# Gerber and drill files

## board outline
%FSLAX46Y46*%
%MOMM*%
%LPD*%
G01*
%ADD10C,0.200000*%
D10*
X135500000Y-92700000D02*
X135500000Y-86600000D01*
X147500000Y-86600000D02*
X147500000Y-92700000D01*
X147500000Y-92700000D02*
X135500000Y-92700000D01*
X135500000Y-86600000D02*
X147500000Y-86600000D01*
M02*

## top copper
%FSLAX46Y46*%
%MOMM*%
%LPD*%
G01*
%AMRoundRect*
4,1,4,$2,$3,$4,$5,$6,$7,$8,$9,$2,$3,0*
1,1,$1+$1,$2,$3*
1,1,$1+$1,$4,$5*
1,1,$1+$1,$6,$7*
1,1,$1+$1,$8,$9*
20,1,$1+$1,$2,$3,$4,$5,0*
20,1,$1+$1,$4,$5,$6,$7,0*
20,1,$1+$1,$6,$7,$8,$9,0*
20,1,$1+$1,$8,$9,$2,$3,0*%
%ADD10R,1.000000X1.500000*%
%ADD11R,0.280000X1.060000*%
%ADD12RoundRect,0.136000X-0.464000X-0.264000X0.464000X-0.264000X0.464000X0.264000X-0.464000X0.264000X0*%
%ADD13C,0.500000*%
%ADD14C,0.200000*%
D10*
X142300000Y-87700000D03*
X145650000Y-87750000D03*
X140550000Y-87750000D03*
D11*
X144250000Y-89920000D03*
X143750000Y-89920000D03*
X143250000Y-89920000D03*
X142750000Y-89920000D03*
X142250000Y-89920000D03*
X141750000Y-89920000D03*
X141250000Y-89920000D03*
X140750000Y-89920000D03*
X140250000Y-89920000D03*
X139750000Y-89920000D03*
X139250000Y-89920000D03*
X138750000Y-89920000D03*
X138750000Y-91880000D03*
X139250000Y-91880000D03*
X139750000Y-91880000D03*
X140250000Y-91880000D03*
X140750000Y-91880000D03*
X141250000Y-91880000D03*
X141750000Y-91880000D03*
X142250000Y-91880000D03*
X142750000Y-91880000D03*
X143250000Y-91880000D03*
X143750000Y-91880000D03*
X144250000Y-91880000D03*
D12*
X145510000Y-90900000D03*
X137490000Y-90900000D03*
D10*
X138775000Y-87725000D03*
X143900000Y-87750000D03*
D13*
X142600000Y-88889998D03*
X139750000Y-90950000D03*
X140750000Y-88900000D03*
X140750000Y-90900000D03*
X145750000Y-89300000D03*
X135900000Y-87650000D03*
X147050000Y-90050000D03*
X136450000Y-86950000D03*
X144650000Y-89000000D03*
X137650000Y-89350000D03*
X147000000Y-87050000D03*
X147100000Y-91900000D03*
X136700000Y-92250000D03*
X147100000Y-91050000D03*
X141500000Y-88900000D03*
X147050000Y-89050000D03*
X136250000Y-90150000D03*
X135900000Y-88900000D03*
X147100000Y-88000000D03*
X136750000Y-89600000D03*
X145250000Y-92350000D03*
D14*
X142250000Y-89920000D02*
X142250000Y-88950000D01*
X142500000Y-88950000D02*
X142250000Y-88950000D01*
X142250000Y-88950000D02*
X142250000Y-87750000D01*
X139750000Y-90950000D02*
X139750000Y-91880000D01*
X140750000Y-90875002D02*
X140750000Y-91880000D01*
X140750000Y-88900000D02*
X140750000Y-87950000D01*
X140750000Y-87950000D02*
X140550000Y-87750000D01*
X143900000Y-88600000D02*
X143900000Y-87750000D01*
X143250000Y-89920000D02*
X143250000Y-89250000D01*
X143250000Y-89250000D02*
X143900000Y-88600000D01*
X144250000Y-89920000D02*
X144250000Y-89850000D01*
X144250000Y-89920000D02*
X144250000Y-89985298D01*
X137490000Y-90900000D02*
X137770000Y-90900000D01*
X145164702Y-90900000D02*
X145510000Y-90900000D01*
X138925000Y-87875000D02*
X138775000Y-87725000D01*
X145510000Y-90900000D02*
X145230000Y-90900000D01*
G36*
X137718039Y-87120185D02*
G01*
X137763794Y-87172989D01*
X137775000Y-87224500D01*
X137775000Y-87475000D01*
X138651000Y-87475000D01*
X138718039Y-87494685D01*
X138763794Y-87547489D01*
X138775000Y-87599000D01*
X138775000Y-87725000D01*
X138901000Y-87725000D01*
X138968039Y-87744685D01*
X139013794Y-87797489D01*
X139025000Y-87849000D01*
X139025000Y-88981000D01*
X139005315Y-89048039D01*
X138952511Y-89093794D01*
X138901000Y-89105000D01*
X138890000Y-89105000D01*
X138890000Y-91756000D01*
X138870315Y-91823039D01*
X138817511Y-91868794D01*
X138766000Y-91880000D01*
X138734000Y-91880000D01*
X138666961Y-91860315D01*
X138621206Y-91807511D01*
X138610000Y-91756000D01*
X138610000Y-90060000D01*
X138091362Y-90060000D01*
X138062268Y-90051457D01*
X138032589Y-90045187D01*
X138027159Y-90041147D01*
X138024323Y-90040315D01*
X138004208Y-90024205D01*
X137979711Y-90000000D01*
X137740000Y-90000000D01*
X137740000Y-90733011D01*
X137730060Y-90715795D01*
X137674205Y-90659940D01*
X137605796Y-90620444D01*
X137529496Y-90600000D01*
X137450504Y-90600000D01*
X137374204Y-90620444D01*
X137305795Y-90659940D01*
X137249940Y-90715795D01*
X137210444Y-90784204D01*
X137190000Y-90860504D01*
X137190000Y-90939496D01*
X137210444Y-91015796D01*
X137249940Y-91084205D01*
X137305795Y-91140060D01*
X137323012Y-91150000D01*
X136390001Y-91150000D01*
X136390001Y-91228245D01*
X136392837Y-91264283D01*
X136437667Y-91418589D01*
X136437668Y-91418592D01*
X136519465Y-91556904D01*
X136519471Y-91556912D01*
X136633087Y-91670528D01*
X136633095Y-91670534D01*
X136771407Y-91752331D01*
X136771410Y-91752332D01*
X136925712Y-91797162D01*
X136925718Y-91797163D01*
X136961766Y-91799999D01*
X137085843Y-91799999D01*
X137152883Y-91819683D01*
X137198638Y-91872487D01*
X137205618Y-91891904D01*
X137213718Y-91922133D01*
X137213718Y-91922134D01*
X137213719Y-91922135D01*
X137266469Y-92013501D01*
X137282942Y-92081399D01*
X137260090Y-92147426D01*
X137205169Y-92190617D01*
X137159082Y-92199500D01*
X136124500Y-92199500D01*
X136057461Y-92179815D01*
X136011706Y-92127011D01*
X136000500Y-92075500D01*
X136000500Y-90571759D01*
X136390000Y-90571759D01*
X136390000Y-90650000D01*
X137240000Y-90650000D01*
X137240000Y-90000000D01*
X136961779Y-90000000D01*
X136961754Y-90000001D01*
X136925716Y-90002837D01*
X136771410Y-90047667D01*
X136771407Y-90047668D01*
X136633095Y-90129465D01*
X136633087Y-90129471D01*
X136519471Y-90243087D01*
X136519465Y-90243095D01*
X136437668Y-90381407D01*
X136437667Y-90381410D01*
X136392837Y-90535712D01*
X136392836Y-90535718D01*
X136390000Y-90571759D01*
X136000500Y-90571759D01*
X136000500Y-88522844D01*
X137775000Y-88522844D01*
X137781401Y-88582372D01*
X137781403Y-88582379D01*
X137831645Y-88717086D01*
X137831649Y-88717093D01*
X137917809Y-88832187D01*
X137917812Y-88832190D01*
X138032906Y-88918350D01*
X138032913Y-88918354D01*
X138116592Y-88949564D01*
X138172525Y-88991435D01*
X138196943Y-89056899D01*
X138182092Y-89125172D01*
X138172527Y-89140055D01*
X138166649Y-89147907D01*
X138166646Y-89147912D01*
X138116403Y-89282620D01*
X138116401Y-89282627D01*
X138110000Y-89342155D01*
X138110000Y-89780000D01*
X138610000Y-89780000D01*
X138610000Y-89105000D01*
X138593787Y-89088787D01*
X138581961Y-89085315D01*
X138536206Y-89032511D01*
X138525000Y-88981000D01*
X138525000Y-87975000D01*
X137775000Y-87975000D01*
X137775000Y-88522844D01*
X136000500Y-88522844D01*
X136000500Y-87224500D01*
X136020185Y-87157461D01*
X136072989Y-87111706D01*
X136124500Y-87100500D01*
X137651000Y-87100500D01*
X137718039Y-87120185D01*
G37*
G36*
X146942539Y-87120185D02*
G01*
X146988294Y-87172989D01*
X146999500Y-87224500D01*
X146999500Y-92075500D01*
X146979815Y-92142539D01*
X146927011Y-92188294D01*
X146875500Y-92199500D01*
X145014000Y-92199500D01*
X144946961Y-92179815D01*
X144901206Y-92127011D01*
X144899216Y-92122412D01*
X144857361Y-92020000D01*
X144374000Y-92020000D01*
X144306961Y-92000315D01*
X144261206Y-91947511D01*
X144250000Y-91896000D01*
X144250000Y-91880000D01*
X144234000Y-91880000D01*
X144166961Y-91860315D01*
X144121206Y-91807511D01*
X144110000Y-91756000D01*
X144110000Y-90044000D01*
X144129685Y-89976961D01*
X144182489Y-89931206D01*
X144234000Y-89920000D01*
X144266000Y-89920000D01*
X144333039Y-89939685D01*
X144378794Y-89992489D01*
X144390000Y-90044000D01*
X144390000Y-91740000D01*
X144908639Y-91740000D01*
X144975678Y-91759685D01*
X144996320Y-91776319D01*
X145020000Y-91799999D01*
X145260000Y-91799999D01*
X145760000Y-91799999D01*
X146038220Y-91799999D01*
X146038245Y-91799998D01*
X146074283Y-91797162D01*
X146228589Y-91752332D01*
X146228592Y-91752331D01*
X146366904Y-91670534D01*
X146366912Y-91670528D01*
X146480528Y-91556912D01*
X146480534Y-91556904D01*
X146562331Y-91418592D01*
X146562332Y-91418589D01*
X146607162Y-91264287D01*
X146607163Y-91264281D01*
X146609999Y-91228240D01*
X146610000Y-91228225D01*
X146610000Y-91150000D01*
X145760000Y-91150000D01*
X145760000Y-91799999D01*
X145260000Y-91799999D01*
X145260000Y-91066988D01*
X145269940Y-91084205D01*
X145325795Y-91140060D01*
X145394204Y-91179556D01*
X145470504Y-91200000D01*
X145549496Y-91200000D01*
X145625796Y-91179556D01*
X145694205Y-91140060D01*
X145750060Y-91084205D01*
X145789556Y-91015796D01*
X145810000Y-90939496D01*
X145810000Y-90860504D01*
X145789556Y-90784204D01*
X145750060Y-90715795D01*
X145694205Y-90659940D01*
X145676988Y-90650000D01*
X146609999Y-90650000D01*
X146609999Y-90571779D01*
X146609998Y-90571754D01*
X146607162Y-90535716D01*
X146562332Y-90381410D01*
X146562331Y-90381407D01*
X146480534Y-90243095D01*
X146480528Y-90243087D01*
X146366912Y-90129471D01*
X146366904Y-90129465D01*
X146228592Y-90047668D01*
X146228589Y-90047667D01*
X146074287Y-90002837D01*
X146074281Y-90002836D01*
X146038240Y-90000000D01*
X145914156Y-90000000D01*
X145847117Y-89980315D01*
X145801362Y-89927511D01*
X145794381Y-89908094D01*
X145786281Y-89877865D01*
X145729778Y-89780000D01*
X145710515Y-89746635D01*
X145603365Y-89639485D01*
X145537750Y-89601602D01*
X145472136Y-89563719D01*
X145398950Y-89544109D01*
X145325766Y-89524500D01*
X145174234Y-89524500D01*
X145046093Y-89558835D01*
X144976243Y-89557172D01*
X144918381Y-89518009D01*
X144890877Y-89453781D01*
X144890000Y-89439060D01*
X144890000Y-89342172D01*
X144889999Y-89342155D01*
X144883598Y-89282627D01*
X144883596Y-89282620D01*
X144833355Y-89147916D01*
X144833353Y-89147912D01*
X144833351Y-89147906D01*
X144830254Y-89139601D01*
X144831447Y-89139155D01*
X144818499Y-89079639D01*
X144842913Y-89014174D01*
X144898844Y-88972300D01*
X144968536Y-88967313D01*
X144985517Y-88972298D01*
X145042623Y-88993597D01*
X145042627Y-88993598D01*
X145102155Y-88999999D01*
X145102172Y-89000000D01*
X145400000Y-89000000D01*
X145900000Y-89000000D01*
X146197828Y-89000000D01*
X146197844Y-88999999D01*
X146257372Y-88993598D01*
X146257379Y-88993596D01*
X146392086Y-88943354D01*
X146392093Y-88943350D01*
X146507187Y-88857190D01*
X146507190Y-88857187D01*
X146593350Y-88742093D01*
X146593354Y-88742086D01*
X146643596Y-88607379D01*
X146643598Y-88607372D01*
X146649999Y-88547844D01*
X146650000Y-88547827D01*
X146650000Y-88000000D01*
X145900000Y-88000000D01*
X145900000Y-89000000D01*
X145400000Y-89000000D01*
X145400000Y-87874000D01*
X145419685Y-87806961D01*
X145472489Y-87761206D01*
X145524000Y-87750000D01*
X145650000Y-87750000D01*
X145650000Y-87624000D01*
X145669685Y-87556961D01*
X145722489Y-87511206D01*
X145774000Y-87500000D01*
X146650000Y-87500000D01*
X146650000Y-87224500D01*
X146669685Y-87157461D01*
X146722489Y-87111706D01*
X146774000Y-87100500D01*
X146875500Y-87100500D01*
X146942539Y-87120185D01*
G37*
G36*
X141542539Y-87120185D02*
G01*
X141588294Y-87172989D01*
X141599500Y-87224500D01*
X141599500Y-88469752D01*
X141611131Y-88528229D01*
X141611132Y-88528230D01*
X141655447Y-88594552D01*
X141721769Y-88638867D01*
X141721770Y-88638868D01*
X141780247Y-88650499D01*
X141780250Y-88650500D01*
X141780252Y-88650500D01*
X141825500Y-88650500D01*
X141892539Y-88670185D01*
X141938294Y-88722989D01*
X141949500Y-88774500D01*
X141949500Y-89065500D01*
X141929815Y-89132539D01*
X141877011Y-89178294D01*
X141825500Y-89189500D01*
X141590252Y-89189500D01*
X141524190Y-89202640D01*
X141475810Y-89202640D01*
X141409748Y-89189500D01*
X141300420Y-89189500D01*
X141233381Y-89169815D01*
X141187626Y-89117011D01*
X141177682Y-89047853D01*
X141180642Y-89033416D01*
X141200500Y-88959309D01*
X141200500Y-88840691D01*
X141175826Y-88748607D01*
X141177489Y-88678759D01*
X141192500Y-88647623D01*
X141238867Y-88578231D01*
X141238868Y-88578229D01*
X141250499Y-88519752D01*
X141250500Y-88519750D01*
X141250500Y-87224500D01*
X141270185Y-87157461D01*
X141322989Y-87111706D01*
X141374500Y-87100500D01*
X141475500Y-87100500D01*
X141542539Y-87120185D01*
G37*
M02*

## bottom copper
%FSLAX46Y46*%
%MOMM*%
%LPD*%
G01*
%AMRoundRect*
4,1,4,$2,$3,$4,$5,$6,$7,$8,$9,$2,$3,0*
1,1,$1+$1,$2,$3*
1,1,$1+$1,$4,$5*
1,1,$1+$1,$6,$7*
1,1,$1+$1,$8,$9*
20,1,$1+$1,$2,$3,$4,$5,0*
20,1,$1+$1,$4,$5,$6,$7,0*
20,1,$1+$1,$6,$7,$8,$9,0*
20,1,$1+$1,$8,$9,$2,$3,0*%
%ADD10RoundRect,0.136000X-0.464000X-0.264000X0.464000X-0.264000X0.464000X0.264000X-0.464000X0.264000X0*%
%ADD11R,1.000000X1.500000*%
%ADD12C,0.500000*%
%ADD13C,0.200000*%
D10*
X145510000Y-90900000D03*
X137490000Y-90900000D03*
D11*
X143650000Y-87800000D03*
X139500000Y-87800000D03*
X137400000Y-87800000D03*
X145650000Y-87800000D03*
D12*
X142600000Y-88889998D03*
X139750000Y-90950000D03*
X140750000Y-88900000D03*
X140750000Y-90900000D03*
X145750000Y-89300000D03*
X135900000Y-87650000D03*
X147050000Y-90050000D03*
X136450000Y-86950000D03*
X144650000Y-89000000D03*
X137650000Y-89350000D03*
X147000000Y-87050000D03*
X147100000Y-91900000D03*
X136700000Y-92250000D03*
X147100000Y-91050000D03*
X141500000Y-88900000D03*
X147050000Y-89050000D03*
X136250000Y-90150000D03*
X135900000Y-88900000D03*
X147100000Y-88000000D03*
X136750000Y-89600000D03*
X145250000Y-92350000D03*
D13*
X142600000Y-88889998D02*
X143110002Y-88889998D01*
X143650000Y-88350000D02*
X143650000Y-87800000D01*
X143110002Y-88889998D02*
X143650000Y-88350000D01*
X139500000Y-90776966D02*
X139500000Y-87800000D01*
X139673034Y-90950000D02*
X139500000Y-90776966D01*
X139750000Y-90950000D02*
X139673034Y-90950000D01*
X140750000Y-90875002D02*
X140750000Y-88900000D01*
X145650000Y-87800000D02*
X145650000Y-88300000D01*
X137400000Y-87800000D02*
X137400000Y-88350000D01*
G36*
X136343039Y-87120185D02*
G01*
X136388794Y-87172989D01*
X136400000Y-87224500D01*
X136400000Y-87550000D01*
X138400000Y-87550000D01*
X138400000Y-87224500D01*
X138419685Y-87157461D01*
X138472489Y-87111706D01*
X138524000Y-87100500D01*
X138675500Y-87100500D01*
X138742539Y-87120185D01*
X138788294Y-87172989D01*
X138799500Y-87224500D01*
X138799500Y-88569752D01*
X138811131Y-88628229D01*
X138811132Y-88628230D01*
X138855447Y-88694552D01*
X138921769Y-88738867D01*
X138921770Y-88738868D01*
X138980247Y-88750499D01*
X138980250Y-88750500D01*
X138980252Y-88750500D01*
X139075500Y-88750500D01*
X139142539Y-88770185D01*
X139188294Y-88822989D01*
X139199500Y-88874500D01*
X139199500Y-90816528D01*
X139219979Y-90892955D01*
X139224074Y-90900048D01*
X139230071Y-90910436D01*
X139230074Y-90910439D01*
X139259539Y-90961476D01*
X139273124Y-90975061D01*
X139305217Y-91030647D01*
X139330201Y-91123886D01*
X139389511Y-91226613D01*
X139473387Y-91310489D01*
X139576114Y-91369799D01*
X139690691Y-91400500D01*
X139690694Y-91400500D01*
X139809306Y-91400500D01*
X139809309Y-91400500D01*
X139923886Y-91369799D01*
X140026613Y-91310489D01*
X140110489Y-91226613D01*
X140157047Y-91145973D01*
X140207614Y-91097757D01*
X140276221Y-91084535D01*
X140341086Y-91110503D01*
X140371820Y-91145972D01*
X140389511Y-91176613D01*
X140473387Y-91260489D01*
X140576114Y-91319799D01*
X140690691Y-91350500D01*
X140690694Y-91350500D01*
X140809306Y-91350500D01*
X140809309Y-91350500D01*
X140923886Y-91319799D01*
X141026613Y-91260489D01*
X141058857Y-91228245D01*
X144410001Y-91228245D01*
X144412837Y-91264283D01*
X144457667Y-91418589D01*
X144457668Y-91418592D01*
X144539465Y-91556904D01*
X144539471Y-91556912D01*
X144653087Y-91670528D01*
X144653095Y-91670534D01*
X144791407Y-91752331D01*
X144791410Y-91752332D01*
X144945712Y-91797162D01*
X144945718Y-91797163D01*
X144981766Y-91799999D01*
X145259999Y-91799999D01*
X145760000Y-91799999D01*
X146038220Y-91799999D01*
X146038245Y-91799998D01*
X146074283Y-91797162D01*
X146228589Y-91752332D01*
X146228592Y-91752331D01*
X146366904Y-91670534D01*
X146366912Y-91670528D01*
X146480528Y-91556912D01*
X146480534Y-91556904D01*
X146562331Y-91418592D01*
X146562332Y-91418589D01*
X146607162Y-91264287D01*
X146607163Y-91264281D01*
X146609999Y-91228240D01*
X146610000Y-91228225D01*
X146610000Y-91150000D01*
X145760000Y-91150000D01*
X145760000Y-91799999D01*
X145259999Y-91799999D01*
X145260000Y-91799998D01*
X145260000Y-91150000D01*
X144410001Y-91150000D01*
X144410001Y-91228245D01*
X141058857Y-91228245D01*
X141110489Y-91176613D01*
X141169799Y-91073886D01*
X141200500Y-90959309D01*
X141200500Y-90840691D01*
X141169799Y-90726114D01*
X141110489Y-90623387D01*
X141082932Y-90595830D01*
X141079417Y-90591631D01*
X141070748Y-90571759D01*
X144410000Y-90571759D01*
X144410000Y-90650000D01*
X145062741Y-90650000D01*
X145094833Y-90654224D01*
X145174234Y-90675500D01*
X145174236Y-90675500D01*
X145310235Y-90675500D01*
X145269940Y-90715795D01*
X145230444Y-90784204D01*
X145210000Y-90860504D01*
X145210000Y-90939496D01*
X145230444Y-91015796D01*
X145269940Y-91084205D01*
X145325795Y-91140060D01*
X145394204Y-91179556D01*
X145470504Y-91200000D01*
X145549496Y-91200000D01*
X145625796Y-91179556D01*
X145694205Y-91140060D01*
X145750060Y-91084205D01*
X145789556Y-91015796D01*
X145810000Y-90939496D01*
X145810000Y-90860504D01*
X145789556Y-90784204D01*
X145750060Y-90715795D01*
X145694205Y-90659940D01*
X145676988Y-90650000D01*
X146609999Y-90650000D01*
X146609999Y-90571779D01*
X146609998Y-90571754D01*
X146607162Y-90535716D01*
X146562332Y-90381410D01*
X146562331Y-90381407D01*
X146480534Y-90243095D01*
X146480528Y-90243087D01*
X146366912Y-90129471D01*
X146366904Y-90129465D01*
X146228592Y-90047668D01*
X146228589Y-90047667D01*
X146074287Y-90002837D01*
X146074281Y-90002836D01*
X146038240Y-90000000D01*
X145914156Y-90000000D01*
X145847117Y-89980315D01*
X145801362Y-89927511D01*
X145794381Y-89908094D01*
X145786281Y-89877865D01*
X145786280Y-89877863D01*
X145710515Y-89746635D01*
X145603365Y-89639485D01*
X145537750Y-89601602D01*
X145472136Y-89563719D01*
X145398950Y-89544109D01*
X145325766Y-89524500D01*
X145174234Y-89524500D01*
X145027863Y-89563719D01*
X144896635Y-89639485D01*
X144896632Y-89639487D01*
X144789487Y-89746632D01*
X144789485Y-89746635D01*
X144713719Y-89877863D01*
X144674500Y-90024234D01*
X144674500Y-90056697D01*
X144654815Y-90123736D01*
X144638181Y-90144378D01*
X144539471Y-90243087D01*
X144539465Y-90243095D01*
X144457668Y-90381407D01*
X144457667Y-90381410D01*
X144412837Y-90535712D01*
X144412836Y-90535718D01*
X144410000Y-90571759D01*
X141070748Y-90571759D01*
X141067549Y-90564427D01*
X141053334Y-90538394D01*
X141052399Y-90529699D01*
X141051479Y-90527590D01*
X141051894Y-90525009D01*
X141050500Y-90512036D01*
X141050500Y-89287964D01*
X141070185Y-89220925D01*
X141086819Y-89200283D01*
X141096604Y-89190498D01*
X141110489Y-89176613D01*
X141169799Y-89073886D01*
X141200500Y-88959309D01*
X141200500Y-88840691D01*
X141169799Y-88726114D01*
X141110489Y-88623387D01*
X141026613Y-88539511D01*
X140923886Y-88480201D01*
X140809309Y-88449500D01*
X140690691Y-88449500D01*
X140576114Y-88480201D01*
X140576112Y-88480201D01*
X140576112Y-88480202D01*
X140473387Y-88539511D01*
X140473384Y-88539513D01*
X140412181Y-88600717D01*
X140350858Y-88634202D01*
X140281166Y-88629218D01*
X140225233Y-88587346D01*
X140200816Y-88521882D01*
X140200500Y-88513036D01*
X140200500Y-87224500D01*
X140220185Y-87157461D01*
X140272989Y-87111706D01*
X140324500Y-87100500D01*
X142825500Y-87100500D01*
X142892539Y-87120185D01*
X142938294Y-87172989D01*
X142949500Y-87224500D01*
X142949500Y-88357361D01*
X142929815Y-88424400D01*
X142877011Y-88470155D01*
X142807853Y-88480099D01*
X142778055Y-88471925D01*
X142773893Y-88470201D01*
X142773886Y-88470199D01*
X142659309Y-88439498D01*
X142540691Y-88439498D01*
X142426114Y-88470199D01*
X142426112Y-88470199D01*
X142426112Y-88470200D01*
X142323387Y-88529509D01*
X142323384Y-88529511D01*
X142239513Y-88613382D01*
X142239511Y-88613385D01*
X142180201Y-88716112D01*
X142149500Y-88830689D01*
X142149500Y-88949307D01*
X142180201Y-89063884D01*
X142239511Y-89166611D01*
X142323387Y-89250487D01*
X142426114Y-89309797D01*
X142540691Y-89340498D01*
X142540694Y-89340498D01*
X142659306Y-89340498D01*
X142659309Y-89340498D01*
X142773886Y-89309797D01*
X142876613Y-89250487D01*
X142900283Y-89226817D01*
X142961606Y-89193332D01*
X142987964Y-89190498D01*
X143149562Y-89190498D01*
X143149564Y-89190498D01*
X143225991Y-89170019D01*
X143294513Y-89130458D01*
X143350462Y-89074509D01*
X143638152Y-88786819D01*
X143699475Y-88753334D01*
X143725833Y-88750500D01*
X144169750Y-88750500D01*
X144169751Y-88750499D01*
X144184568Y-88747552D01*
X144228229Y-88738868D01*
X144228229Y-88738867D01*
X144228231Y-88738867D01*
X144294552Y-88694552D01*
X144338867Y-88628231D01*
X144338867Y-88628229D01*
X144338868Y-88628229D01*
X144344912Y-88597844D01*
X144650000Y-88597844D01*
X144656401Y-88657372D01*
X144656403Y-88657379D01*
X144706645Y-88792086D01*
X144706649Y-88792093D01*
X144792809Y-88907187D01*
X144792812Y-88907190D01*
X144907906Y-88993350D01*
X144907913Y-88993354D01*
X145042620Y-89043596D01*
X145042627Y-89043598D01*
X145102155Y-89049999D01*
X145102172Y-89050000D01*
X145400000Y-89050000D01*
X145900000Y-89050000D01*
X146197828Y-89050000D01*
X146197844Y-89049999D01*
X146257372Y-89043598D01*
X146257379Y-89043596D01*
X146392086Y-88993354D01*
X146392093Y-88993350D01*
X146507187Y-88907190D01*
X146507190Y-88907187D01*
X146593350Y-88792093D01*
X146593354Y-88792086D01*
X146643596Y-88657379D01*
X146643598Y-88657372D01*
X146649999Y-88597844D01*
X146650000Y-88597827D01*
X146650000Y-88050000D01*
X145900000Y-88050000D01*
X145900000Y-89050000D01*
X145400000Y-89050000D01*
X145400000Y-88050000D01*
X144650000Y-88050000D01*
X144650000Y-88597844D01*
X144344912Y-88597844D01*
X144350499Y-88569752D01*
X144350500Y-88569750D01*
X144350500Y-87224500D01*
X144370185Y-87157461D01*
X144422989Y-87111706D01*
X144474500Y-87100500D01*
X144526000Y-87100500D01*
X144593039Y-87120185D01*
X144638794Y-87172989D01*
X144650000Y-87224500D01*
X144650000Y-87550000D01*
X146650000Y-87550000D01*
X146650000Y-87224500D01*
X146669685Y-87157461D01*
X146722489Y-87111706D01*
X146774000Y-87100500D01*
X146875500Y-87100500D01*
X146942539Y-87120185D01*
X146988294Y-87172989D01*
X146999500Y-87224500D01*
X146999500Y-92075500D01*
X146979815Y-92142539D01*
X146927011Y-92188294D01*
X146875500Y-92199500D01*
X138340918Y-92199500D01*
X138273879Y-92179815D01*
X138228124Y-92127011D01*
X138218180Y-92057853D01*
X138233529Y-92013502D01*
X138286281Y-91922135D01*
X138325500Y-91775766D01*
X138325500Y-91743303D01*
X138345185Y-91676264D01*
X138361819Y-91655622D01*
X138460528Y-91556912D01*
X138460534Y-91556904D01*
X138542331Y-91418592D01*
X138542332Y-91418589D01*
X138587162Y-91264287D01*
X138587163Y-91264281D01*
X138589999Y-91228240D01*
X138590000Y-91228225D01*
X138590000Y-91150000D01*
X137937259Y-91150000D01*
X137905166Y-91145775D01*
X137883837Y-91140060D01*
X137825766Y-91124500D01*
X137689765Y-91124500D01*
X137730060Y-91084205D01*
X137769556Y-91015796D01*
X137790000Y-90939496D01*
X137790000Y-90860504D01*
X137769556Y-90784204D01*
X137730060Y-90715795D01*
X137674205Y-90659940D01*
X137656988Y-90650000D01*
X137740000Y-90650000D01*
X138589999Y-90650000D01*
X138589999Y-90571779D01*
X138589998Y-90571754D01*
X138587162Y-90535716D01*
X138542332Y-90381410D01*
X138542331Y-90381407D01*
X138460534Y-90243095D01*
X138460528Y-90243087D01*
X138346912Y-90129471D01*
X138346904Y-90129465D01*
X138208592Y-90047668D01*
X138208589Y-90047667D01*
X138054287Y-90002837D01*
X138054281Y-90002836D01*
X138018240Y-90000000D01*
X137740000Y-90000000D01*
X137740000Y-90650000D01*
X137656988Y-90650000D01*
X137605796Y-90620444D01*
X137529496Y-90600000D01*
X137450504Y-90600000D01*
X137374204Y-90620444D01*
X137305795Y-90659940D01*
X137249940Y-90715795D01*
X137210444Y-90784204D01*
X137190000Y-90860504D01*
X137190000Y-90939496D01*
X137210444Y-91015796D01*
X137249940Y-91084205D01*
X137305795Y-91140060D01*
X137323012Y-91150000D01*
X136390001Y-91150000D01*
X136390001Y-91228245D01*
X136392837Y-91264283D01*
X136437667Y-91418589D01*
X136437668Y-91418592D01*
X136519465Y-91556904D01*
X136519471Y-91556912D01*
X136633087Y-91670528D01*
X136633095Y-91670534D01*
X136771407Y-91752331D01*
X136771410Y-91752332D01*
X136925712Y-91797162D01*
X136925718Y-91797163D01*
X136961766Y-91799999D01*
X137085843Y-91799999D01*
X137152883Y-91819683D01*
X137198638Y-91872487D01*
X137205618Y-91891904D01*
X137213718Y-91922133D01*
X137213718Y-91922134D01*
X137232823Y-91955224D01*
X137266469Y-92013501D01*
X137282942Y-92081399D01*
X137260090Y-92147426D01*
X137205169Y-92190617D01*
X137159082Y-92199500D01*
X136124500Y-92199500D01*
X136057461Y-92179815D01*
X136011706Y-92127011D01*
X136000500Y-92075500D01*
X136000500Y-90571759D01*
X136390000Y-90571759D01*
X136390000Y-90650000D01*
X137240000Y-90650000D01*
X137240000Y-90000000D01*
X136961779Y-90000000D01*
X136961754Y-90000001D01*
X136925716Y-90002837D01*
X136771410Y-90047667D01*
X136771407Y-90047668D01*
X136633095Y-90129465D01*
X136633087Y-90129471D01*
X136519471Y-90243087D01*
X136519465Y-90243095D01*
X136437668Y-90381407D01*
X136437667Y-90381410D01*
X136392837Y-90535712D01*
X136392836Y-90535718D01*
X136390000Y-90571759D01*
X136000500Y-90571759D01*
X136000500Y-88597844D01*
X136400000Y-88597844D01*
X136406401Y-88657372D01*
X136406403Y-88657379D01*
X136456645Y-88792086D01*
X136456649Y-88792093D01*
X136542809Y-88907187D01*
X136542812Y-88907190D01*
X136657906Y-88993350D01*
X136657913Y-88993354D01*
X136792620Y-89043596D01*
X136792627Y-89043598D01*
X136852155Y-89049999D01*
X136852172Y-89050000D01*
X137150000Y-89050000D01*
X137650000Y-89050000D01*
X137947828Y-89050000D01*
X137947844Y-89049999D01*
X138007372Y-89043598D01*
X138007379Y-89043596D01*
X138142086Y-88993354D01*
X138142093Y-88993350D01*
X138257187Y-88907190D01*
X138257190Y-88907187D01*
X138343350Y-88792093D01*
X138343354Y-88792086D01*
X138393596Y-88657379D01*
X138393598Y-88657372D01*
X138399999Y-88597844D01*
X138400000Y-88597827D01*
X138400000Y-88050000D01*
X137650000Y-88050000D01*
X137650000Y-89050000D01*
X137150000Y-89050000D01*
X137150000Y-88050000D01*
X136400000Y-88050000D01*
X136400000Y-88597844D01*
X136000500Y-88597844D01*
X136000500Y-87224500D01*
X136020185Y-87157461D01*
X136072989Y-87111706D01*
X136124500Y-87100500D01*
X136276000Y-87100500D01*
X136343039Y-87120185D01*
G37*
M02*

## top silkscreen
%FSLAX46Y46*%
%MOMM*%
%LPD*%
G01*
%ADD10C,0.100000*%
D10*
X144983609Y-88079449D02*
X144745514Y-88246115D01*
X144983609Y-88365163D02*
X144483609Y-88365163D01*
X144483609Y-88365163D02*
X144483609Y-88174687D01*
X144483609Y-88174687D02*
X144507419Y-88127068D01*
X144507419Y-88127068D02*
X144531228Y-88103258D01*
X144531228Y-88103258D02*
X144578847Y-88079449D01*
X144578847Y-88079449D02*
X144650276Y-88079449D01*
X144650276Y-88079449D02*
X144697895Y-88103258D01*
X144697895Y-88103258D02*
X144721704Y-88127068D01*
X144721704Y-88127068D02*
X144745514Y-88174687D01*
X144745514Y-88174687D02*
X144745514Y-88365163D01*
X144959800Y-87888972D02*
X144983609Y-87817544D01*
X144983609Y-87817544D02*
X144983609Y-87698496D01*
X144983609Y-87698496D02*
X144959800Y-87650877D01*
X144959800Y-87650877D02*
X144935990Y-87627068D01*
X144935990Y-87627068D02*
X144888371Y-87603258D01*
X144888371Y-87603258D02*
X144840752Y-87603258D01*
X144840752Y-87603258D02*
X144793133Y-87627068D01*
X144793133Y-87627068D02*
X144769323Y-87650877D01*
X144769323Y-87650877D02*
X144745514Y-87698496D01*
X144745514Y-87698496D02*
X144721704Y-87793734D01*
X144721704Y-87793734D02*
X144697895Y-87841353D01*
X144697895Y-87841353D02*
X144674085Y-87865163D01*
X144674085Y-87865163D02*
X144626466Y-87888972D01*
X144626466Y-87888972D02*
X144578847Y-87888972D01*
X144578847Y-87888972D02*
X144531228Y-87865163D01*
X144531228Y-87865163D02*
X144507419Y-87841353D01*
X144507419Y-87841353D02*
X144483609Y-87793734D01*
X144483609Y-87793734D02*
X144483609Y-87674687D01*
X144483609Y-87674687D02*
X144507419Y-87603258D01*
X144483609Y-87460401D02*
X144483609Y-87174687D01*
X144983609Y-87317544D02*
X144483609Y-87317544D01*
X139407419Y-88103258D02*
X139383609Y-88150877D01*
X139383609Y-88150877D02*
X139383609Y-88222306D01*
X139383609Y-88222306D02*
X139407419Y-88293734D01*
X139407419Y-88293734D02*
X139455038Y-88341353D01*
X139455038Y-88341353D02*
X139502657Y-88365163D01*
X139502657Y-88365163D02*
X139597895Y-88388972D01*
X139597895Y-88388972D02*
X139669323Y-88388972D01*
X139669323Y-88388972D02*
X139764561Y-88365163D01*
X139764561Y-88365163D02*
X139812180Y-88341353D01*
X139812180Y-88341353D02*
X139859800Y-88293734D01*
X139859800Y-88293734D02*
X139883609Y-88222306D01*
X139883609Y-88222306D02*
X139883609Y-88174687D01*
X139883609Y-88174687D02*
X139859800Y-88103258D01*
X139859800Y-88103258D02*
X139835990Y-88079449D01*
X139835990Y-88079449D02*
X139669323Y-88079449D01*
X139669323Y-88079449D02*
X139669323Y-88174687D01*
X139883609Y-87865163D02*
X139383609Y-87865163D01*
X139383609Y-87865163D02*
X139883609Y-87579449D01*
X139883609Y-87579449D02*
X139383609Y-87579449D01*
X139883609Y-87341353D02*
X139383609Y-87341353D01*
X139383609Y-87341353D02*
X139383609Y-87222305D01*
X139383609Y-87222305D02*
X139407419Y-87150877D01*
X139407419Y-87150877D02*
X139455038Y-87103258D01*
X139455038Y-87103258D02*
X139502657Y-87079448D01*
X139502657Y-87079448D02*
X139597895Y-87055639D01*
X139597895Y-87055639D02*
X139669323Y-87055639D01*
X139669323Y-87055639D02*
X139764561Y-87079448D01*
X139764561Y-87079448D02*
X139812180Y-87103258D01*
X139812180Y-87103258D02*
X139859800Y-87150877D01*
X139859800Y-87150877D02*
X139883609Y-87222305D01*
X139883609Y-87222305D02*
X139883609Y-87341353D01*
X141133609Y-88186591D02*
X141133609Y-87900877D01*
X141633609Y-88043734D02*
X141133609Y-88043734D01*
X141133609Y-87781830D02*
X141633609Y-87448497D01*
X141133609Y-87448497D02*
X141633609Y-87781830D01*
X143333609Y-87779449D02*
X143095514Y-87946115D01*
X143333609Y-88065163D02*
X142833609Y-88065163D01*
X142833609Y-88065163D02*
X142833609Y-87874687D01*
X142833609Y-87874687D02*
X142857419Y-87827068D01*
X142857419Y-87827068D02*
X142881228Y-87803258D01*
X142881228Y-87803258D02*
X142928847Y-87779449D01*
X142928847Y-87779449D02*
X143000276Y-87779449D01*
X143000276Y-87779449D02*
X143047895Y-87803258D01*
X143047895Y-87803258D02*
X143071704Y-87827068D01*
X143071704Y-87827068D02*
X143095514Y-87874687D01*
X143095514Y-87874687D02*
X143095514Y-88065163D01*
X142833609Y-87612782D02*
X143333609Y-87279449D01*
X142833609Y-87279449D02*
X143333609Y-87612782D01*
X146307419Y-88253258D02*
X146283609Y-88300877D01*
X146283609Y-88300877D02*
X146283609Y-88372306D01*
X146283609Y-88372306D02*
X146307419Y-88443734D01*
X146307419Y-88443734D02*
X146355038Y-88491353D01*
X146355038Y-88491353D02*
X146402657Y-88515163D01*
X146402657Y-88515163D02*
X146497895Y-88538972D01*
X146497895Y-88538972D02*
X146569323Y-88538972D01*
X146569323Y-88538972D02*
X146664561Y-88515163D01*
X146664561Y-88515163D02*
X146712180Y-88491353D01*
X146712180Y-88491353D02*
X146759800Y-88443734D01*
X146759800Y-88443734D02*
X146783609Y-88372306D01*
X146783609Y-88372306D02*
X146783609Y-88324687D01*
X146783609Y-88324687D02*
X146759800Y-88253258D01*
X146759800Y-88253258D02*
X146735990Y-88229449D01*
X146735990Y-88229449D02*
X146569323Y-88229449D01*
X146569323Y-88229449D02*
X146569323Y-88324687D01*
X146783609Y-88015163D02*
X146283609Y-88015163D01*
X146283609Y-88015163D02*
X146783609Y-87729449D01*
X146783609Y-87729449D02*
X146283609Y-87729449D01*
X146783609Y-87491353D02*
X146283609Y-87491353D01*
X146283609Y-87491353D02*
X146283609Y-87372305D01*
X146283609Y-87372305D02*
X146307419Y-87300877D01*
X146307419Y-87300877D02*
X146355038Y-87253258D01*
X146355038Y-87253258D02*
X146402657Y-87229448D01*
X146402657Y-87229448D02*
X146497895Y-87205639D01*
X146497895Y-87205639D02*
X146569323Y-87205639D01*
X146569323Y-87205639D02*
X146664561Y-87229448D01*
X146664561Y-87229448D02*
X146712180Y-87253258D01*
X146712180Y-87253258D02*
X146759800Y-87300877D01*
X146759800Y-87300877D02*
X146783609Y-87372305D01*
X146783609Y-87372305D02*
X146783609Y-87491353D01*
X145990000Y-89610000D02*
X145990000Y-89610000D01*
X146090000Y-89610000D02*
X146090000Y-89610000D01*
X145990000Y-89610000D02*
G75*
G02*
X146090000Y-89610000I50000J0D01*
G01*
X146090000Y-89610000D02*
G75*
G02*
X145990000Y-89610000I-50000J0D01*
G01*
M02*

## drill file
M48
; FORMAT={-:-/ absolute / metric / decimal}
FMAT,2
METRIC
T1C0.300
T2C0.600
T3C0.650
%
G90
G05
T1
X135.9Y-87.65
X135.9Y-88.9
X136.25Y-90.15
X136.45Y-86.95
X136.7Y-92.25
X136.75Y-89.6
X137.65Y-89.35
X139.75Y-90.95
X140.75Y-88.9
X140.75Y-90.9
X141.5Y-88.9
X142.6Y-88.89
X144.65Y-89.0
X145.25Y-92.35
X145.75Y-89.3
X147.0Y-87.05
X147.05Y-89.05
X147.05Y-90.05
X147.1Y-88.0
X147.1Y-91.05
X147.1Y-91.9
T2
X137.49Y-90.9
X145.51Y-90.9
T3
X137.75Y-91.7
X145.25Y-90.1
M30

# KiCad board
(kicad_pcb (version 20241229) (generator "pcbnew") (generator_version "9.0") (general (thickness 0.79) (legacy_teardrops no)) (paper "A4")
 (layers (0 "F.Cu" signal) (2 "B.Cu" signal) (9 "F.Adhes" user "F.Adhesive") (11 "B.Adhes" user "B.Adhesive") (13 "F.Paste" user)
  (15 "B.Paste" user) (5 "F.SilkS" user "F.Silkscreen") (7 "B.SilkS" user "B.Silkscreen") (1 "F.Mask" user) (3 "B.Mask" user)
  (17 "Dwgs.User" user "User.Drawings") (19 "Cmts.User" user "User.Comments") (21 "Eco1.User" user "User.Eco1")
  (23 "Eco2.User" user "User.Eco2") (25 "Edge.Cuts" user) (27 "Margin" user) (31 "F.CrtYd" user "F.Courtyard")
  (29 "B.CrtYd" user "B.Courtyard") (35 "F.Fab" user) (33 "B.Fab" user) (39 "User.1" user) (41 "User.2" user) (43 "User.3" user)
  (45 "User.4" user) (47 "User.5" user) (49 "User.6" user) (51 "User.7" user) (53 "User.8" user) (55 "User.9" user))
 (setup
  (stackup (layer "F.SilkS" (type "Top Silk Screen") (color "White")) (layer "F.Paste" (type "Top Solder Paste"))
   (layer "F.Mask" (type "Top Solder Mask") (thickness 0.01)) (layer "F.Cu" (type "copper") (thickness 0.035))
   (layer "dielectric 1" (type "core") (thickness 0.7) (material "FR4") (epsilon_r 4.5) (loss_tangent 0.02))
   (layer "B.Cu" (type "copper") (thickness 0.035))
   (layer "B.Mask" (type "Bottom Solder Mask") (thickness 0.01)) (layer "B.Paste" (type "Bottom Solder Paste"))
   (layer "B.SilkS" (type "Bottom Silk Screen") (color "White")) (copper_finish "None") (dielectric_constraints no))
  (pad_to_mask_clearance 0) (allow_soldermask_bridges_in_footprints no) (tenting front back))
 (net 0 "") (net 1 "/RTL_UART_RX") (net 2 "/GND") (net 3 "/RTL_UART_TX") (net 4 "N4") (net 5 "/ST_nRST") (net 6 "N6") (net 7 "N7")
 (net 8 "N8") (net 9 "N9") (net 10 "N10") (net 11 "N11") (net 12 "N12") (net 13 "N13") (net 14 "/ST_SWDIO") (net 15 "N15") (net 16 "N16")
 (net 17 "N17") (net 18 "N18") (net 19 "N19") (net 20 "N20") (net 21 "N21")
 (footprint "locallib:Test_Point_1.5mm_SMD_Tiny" (layer "F.Cu") (at 142.3 87.7)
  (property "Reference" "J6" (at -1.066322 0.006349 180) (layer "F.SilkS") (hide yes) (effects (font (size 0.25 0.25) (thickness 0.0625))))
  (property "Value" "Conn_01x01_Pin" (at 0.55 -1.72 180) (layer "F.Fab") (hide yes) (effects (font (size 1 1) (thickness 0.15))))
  (pad "1" smd rect (at 0 0) (size 1 1.5) (layers "F.Cu" "F.Mask") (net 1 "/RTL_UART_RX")))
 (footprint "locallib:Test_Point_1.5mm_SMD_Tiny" (layer "F.Cu") (at 145.65 87.75)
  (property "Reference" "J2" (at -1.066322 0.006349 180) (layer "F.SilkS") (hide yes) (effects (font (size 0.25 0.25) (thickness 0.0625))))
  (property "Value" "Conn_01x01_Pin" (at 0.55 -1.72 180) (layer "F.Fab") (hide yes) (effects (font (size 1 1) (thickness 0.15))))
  (pad "1" smd rect (at 0 0) (size 1 1.5) (layers "F.Cu" "F.Mask") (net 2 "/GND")))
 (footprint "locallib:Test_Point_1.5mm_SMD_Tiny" (layer "F.Cu") (at 140.55 87.75)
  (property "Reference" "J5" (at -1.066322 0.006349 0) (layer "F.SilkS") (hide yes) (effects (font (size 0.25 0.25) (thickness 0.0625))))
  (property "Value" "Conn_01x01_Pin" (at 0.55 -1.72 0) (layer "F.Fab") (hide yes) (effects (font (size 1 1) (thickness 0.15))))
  (pad "1" smd rect (at 0 0) (size 1 1.5) (layers "F.Cu" "F.Mask") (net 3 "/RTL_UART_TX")))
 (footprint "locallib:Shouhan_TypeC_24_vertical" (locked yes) (layer "F.Cu") (at 141.5 91)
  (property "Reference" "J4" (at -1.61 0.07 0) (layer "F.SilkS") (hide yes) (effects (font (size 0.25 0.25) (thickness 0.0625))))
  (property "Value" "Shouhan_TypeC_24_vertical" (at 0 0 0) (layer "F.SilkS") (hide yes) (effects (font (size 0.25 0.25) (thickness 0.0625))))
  (fp_line (start 4.49 -1.39) (end 4.49 -1.39) (stroke (width 0.1) (type solid)) (layer "F.SilkS"))
  (fp_line (start 4.59 -1.39) (end 4.59 -1.39) (stroke (width 0.1) (type solid)) (layer "F.SilkS"))
  (fp_arc (start 4.49 -1.39) (mid 4.54 -1.44) (end 4.59 -1.39) (stroke (width 0.1) (type solid)) (layer "F.SilkS"))
  (fp_arc (start 4.59 -1.39) (mid 4.54 -1.34) (end 4.49 -1.39) (stroke (width 0.1) (type solid)) (layer "F.SilkS"))
  (pad "" np_thru_hole circle (at -3.75 0.7) (size 0.5 0.5) (drill 0.65) (layers "*.Cu" "*.Mask"))
  (pad "" np_thru_hole circle (at 3.75 -0.9) (size 0.5 0.5) (drill 0.65) (layers "*.Cu" "*.Mask"))
  (pad "A1" smd rect (at 2.75 -1.08) (size 0.28 1.06) (layers "F.Cu" "F.Mask" "F.Paste") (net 2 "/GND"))
  (pad "A2" smd rect (at 2.25 -1.08) (size 0.28 1.06) (layers "F.Cu" "F.Mask" "F.Paste") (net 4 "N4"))
  (pad "A3" smd rect (at 1.75 -1.08) (size 0.28 1.06) (layers "F.Cu" "F.Mask" "F.Paste") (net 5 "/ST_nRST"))
  (pad "A4" smd rect (at 1.25 -1.08) (size 0.28 1.06) (layers "F.Cu" "F.Mask" "F.Paste") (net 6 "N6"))
  (pad "A5" smd rect (at 0.75 -1.08) (size 0.28 1.06) (layers "F.Cu" "F.Mask" "F.Paste") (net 1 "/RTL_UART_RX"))
  (pad "A6" smd rect (at 0.25 -1.08) (size 0.28 1.06) (layers "F.Cu" "F.Mask" "F.Paste") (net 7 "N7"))
  (pad "A7" smd rect (at -0.25 -1.08) (size 0.28 1.06) (layers "F.Cu" "F.Mask" "F.Paste") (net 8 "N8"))
  (pad "A8" smd rect (at -0.75 -1.08) (size 0.28 1.06) (layers "F.Cu" "F.Mask" "F.Paste") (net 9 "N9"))
  (pad "A9" smd rect (at -1.25 -1.08) (size 0.28 1.06) (layers "F.Cu" "F.Mask" "F.Paste") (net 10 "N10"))
  (pad "A10" smd rect (at -1.75 -1.08) (size 0.28 1.06) (layers "F.Cu" "F.Mask" "F.Paste") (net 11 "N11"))
  (pad "A11" smd rect (at -2.25 -1.08) (size 0.28 1.06) (layers "F.Cu" "F.Mask" "F.Paste") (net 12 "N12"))
  (pad "A12" smd rect (at -2.75 -1.08) (size 0.28 1.06) (layers "F.Cu" "F.Mask" "F.Paste") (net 2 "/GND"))
  (pad "B1" smd rect (at -2.75 0.88) (size 0.28 1.06) (layers "F.Cu" "F.Mask" "F.Paste") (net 2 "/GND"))
  (pad "B2" smd rect (at -2.25 0.88) (size 0.28 1.06) (layers "F.Cu" "F.Mask" "F.Paste") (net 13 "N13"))
  (pad "B3" smd rect (at -1.75 0.88) (size 0.28 1.06) (layers "F.Cu" "F.Mask" "F.Paste") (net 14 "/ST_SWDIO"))
  (pad "B4" smd rect (at -1.25 0.88) (size 0.28 1.06) (layers "F.Cu" "F.Mask" "F.Paste") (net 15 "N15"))
  (pad "B5" smd rect (at -0.75 0.88) (size 0.28 1.06) (layers "F.Cu" "F.Mask" "F.Paste") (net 3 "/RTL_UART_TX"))
  (pad "B6" smd rect (at -0.25 0.88) (size 0.28 1.06) (layers "F.Cu" "F.Mask" "F.Paste") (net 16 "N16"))
  (pad "B7" smd rect (at 0.25 0.88) (size 0.28 1.06) (layers "F.Cu" "F.Mask" "F.Paste") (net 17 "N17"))
  (pad "B8" smd rect (at 0.75 0.88) (size 0.28 1.06) (layers "F.Cu" "F.Mask" "F.Paste") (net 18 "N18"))
  (pad "B9" smd rect (at 1.25 0.88) (size 0.28 1.06) (layers "F.Cu" "F.Mask" "F.Paste") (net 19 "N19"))
  (pad "B10" smd rect (at 1.75 0.88) (size 0.28 1.06) (layers "F.Cu" "F.Mask" "F.Paste") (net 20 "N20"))
  (pad "B11" smd rect (at 2.25 0.88) (size 0.28 1.06) (layers "F.Cu" "F.Mask" "F.Paste") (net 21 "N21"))
  (pad "B12" smd rect (at 2.75 0.88) (size 0.28 1.06) (layers "F.Cu" "F.Mask" "F.Paste") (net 2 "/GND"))
  (pad "MH1" thru_hole roundrect (at 4.01 -0.1) (size 1.2 0.8) (drill 0.6) (layers "*.Cu" "*.Mask") (remove_unused_layers no)
   (roundrect_rratio 0.17) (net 2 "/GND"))
  (pad "MH2" thru_hole roundrect (at -4.01 -0.1) (size 1.2 0.8) (drill 0.6) (layers "*.Cu" "*.Mask") (remove_unused_layers no)
   (roundrect_rratio 0.17) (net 2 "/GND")))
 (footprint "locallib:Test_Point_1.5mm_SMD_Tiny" (layer "F.Cu") (at 138.775 87.725)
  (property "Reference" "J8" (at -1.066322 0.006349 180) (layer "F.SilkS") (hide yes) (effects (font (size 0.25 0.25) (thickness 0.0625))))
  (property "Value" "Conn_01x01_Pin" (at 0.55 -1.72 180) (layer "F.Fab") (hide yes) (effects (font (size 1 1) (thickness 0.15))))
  (pad "1" smd rect (at 0 0) (size 1 1.5) (layers "F.Cu" "F.Mask") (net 2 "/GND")))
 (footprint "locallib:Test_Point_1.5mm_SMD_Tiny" (layer "F.Cu") (at 143.9 87.75)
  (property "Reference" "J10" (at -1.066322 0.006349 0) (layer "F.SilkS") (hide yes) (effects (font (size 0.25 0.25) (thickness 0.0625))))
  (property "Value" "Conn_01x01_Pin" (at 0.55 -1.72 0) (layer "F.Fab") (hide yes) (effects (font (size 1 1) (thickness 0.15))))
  (pad "1" smd rect (at 0 0) (size 1 1.5) (layers "F.Cu" "F.Mask") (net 5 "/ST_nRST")))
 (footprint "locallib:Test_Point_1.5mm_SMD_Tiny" (layer "B.Cu") (at 143.65 87.8 180)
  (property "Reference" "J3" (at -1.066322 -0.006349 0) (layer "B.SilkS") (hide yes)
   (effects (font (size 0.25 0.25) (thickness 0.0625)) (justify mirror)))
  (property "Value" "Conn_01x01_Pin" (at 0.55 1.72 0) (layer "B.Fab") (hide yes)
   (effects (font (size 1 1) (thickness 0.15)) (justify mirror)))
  (pad "1" smd rect (at 0 0 180) (size 1 1.5) (layers "B.Cu" "B.Mask") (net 1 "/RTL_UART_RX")))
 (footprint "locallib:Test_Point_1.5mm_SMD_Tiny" (layer "B.Cu") (at 139.5 87.8 180)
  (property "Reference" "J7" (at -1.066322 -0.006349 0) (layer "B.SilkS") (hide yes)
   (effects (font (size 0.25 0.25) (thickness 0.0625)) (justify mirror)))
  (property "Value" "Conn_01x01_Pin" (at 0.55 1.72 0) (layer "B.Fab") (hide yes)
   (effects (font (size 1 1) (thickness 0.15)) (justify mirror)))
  (pad "1" smd rect (at 0 0 180) (size 1 1.5) (layers "B.Cu" "B.Mask") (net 14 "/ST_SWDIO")))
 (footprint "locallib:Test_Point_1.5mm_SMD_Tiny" (layer "B.Cu") (at 137.4 87.8 180)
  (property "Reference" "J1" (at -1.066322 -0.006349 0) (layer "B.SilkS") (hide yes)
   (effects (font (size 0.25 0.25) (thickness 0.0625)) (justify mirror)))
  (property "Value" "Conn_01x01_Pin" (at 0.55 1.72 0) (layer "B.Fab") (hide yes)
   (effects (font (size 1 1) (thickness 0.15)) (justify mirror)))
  (pad "1" smd rect (at 0 0 180) (size 1 1.5) (layers "B.Cu" "B.Mask") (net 2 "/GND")))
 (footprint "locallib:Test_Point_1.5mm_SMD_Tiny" (layer "B.Cu") (at 145.65 87.8 180)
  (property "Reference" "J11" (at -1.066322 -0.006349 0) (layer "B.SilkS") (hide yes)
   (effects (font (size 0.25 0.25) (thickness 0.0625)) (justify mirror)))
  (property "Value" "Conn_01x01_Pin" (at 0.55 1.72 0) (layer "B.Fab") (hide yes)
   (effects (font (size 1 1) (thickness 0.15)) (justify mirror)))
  (pad "1" smd rect (at 0 0 180) (size 1 1.5) (layers "B.Cu" "B.Mask") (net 2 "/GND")))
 (gr_line (start 135.5 92.7) (end 135.5 86.6) (stroke (width 0.2) (type solid)) (locked yes) (layer "Edge.Cuts"))
 (gr_line (start 147.5 86.6) (end 147.5 92.7) (stroke (width 0.2) (type solid)) (locked yes) (layer "Edge.Cuts"))
 (gr_line (start 147.5 92.7) (end 135.5 92.7) (stroke (width 0.2) (type solid)) (locked yes) (layer "Edge.Cuts"))
 (gr_line (start 135.5 86.6) (end 147.5 86.6) (stroke (width 0.2) (type solid)) (locked yes) (layer "Edge.Cuts"))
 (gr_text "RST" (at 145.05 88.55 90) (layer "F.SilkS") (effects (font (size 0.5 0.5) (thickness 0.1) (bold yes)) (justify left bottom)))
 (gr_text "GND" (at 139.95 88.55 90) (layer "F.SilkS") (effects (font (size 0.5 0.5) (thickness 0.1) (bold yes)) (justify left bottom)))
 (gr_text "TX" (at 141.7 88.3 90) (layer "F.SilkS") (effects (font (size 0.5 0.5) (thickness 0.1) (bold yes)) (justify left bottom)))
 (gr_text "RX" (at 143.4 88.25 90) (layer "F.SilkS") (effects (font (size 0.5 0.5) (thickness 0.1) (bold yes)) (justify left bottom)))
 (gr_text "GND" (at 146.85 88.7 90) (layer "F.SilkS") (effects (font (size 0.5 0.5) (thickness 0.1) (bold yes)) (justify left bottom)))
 (segment (start 142.25 89.92) (end 142.25 88.95) (width 0.2) (layer "F.Cu") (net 1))
 (segment (start 142.5 88.95) (end 142.25 88.95) (width 0.2) (layer "F.Cu") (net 1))
 (segment (start 142.25 88.95) (end 142.25 87.75) (width 0.2) (layer "F.Cu") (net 1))
 (via (at 142.6 88.889998) (size 0.5) (drill 0.3) (layers "F.Cu" "B.Cu") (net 1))
 (segment (start 142.6 88.889998) (end 143.110002 88.889998) (width 0.2) (layer "B.Cu") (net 1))
 (segment (start 143.65 88.35) (end 143.65 87.8) (width 0.2) (layer "B.Cu") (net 1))
 (segment (start 143.110002 88.889998) (end 143.65 88.35) (width 0.2) (layer "B.Cu") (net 1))
 (segment (start 139.75 90.95) (end 139.75 91.88) (width 0.2) (layer "F.Cu") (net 14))
 (via (at 139.75 90.95) (size 0.5) (drill 0.3) (layers "F.Cu" "B.Cu") (free yes) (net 14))
 (segment (start 139.5 90.776966) (end 139.5 87.8) (width 0.2) (layer "B.Cu") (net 14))
 (segment (start 139.673034 90.95) (end 139.5 90.776966) (width 0.2) (layer "B.Cu") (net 14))
 (segment (start 139.75 90.95) (end 139.673034 90.95) (width 0.2) (layer "B.Cu") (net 14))
 (segment (start 140.75 90.875002) (end 140.75 91.88) (width 0.2) (layer "F.Cu") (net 3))
 (segment (start 140.75 88.9) (end 140.75 87.95) (width 0.2) (layer "F.Cu") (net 3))
 (segment (start 140.75 87.95) (end 140.55 87.75) (width 0.2) (layer "F.Cu") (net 3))
 (via (at 140.75 88.9) (size 0.5) (drill 0.3) (layers "F.Cu" "B.Cu") (free yes) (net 3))
 (via (at 140.75 90.9) (size 0.5) (drill 0.3) (layers "F.Cu" "B.Cu") (free yes) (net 3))
 (segment (start 140.75 90.875002) (end 140.75 88.9) (width 0.2) (layer "B.Cu") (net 3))
 (segment (start 143.9 88.6) (end 143.9 87.75) (width 0.2) (layer "F.Cu") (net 5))
 (segment (start 143.25 89.92) (end 143.25 89.25) (width 0.2) (layer "F.Cu") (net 5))
 (segment (start 143.25 89.25) (end 143.9 88.6) (width 0.2) (layer "F.Cu") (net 5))
 (segment (start 144.25 89.92) (end 144.25 89.85) (width 0.2) (layer "F.Cu") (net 2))
 (segment (start 144.25 89.92) (end 144.25 89.985298) (width 0.2) (layer "F.Cu") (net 2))
 (segment (start 137.49 90.9) (end 137.77 90.9) (width 0.2) (layer "F.Cu") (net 2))
 (segment (start 145.164702 90.9) (end 145.51 90.9) (width 0.2) (layer "F.Cu") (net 2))
 (segment (start 138.925 87.875) (end 138.775 87.725) (width 0.2) (layer "F.Cu") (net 2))
 (segment (start 145.51 90.9) (end 145.23 90.9) (width 0.2) (layer "F.Cu") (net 2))
 (via (at 145.75 89.3) (size 0.5) (drill 0.3) (layers "F.Cu" "B.Cu") (free yes) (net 2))
 (via (at 135.9 87.65) (size 0.5) (drill 0.3) (layers "F.Cu" "B.Cu") (free yes) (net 2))
 (via (at 147.05 90.05) (size 0.5) (drill 0.3) (layers "F.Cu" "B.Cu") (free yes) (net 2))
 (via (at 136.45 86.95) (size 0.5) (drill 0.3) (layers "F.Cu" "B.Cu") (free yes) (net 2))
 (via (at 144.65 89) (size 0.5) (drill 0.3) (layers "F.Cu" "B.Cu") (free yes) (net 2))
 (via (at 137.65 89.35) (size 0.5) (drill 0.3) (layers "F.Cu" "B.Cu") (free yes) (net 2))
 (via (at 147 87.05) (size 0.5) (drill 0.3) (layers "F.Cu" "B.Cu") (free yes) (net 2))
 (via (at 147.1 91.9) (size 0.5) (drill 0.3) (layers "F.Cu" "B.Cu") (free yes) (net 2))
 (via (at 136.7 92.25) (size 0.5) (drill 0.3) (layers "F.Cu" "B.Cu") (free yes) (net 2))
 (via (at 147.1 91.05) (size 0.5) (drill 0.3) (layers "F.Cu" "B.Cu") (free yes) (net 2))
 (via (at 141.5 88.9) (size 0.5) (drill 0.3) (layers "F.Cu" "B.Cu") (free yes) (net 2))
 (via (at 147.05 89.05) (size 0.5) (drill 0.3) (layers "F.Cu" "B.Cu") (free yes) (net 2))
 (via (at 136.25 90.15) (size 0.5) (drill 0.3) (layers "F.Cu" "B.Cu") (free yes) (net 2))
 (via (at 135.9 88.9) (size 0.5) (drill 0.3) (layers "F.Cu" "B.Cu") (free yes) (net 2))
 (via (at 147.1 88) (size 0.5) (drill 0.3) (layers "F.Cu" "B.Cu") (free yes) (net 2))
 (via (at 136.75 89.6) (size 0.5) (drill 0.3) (layers "F.Cu" "B.Cu") (free yes) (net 2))
 (via (at 145.25 92.35) (size 0.5) (drill 0.3) (layers "F.Cu" "B.Cu") (free yes) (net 2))
 (segment (start 145.65 87.8) (end 145.65 88.3) (width 0.2) (layer "B.Cu") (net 2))
 (segment (start 137.4 87.8) (end 137.4 88.35) (width 0.2) (layer "B.Cu") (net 2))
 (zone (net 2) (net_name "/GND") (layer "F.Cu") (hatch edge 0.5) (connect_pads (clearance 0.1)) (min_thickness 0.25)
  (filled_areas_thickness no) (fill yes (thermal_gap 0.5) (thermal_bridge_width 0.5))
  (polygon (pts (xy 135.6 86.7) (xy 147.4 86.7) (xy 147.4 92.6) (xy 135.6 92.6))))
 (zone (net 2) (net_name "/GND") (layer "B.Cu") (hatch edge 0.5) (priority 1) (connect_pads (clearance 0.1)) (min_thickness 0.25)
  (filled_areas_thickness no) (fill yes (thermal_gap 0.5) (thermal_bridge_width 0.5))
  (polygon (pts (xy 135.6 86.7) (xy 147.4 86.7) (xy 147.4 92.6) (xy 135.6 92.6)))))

